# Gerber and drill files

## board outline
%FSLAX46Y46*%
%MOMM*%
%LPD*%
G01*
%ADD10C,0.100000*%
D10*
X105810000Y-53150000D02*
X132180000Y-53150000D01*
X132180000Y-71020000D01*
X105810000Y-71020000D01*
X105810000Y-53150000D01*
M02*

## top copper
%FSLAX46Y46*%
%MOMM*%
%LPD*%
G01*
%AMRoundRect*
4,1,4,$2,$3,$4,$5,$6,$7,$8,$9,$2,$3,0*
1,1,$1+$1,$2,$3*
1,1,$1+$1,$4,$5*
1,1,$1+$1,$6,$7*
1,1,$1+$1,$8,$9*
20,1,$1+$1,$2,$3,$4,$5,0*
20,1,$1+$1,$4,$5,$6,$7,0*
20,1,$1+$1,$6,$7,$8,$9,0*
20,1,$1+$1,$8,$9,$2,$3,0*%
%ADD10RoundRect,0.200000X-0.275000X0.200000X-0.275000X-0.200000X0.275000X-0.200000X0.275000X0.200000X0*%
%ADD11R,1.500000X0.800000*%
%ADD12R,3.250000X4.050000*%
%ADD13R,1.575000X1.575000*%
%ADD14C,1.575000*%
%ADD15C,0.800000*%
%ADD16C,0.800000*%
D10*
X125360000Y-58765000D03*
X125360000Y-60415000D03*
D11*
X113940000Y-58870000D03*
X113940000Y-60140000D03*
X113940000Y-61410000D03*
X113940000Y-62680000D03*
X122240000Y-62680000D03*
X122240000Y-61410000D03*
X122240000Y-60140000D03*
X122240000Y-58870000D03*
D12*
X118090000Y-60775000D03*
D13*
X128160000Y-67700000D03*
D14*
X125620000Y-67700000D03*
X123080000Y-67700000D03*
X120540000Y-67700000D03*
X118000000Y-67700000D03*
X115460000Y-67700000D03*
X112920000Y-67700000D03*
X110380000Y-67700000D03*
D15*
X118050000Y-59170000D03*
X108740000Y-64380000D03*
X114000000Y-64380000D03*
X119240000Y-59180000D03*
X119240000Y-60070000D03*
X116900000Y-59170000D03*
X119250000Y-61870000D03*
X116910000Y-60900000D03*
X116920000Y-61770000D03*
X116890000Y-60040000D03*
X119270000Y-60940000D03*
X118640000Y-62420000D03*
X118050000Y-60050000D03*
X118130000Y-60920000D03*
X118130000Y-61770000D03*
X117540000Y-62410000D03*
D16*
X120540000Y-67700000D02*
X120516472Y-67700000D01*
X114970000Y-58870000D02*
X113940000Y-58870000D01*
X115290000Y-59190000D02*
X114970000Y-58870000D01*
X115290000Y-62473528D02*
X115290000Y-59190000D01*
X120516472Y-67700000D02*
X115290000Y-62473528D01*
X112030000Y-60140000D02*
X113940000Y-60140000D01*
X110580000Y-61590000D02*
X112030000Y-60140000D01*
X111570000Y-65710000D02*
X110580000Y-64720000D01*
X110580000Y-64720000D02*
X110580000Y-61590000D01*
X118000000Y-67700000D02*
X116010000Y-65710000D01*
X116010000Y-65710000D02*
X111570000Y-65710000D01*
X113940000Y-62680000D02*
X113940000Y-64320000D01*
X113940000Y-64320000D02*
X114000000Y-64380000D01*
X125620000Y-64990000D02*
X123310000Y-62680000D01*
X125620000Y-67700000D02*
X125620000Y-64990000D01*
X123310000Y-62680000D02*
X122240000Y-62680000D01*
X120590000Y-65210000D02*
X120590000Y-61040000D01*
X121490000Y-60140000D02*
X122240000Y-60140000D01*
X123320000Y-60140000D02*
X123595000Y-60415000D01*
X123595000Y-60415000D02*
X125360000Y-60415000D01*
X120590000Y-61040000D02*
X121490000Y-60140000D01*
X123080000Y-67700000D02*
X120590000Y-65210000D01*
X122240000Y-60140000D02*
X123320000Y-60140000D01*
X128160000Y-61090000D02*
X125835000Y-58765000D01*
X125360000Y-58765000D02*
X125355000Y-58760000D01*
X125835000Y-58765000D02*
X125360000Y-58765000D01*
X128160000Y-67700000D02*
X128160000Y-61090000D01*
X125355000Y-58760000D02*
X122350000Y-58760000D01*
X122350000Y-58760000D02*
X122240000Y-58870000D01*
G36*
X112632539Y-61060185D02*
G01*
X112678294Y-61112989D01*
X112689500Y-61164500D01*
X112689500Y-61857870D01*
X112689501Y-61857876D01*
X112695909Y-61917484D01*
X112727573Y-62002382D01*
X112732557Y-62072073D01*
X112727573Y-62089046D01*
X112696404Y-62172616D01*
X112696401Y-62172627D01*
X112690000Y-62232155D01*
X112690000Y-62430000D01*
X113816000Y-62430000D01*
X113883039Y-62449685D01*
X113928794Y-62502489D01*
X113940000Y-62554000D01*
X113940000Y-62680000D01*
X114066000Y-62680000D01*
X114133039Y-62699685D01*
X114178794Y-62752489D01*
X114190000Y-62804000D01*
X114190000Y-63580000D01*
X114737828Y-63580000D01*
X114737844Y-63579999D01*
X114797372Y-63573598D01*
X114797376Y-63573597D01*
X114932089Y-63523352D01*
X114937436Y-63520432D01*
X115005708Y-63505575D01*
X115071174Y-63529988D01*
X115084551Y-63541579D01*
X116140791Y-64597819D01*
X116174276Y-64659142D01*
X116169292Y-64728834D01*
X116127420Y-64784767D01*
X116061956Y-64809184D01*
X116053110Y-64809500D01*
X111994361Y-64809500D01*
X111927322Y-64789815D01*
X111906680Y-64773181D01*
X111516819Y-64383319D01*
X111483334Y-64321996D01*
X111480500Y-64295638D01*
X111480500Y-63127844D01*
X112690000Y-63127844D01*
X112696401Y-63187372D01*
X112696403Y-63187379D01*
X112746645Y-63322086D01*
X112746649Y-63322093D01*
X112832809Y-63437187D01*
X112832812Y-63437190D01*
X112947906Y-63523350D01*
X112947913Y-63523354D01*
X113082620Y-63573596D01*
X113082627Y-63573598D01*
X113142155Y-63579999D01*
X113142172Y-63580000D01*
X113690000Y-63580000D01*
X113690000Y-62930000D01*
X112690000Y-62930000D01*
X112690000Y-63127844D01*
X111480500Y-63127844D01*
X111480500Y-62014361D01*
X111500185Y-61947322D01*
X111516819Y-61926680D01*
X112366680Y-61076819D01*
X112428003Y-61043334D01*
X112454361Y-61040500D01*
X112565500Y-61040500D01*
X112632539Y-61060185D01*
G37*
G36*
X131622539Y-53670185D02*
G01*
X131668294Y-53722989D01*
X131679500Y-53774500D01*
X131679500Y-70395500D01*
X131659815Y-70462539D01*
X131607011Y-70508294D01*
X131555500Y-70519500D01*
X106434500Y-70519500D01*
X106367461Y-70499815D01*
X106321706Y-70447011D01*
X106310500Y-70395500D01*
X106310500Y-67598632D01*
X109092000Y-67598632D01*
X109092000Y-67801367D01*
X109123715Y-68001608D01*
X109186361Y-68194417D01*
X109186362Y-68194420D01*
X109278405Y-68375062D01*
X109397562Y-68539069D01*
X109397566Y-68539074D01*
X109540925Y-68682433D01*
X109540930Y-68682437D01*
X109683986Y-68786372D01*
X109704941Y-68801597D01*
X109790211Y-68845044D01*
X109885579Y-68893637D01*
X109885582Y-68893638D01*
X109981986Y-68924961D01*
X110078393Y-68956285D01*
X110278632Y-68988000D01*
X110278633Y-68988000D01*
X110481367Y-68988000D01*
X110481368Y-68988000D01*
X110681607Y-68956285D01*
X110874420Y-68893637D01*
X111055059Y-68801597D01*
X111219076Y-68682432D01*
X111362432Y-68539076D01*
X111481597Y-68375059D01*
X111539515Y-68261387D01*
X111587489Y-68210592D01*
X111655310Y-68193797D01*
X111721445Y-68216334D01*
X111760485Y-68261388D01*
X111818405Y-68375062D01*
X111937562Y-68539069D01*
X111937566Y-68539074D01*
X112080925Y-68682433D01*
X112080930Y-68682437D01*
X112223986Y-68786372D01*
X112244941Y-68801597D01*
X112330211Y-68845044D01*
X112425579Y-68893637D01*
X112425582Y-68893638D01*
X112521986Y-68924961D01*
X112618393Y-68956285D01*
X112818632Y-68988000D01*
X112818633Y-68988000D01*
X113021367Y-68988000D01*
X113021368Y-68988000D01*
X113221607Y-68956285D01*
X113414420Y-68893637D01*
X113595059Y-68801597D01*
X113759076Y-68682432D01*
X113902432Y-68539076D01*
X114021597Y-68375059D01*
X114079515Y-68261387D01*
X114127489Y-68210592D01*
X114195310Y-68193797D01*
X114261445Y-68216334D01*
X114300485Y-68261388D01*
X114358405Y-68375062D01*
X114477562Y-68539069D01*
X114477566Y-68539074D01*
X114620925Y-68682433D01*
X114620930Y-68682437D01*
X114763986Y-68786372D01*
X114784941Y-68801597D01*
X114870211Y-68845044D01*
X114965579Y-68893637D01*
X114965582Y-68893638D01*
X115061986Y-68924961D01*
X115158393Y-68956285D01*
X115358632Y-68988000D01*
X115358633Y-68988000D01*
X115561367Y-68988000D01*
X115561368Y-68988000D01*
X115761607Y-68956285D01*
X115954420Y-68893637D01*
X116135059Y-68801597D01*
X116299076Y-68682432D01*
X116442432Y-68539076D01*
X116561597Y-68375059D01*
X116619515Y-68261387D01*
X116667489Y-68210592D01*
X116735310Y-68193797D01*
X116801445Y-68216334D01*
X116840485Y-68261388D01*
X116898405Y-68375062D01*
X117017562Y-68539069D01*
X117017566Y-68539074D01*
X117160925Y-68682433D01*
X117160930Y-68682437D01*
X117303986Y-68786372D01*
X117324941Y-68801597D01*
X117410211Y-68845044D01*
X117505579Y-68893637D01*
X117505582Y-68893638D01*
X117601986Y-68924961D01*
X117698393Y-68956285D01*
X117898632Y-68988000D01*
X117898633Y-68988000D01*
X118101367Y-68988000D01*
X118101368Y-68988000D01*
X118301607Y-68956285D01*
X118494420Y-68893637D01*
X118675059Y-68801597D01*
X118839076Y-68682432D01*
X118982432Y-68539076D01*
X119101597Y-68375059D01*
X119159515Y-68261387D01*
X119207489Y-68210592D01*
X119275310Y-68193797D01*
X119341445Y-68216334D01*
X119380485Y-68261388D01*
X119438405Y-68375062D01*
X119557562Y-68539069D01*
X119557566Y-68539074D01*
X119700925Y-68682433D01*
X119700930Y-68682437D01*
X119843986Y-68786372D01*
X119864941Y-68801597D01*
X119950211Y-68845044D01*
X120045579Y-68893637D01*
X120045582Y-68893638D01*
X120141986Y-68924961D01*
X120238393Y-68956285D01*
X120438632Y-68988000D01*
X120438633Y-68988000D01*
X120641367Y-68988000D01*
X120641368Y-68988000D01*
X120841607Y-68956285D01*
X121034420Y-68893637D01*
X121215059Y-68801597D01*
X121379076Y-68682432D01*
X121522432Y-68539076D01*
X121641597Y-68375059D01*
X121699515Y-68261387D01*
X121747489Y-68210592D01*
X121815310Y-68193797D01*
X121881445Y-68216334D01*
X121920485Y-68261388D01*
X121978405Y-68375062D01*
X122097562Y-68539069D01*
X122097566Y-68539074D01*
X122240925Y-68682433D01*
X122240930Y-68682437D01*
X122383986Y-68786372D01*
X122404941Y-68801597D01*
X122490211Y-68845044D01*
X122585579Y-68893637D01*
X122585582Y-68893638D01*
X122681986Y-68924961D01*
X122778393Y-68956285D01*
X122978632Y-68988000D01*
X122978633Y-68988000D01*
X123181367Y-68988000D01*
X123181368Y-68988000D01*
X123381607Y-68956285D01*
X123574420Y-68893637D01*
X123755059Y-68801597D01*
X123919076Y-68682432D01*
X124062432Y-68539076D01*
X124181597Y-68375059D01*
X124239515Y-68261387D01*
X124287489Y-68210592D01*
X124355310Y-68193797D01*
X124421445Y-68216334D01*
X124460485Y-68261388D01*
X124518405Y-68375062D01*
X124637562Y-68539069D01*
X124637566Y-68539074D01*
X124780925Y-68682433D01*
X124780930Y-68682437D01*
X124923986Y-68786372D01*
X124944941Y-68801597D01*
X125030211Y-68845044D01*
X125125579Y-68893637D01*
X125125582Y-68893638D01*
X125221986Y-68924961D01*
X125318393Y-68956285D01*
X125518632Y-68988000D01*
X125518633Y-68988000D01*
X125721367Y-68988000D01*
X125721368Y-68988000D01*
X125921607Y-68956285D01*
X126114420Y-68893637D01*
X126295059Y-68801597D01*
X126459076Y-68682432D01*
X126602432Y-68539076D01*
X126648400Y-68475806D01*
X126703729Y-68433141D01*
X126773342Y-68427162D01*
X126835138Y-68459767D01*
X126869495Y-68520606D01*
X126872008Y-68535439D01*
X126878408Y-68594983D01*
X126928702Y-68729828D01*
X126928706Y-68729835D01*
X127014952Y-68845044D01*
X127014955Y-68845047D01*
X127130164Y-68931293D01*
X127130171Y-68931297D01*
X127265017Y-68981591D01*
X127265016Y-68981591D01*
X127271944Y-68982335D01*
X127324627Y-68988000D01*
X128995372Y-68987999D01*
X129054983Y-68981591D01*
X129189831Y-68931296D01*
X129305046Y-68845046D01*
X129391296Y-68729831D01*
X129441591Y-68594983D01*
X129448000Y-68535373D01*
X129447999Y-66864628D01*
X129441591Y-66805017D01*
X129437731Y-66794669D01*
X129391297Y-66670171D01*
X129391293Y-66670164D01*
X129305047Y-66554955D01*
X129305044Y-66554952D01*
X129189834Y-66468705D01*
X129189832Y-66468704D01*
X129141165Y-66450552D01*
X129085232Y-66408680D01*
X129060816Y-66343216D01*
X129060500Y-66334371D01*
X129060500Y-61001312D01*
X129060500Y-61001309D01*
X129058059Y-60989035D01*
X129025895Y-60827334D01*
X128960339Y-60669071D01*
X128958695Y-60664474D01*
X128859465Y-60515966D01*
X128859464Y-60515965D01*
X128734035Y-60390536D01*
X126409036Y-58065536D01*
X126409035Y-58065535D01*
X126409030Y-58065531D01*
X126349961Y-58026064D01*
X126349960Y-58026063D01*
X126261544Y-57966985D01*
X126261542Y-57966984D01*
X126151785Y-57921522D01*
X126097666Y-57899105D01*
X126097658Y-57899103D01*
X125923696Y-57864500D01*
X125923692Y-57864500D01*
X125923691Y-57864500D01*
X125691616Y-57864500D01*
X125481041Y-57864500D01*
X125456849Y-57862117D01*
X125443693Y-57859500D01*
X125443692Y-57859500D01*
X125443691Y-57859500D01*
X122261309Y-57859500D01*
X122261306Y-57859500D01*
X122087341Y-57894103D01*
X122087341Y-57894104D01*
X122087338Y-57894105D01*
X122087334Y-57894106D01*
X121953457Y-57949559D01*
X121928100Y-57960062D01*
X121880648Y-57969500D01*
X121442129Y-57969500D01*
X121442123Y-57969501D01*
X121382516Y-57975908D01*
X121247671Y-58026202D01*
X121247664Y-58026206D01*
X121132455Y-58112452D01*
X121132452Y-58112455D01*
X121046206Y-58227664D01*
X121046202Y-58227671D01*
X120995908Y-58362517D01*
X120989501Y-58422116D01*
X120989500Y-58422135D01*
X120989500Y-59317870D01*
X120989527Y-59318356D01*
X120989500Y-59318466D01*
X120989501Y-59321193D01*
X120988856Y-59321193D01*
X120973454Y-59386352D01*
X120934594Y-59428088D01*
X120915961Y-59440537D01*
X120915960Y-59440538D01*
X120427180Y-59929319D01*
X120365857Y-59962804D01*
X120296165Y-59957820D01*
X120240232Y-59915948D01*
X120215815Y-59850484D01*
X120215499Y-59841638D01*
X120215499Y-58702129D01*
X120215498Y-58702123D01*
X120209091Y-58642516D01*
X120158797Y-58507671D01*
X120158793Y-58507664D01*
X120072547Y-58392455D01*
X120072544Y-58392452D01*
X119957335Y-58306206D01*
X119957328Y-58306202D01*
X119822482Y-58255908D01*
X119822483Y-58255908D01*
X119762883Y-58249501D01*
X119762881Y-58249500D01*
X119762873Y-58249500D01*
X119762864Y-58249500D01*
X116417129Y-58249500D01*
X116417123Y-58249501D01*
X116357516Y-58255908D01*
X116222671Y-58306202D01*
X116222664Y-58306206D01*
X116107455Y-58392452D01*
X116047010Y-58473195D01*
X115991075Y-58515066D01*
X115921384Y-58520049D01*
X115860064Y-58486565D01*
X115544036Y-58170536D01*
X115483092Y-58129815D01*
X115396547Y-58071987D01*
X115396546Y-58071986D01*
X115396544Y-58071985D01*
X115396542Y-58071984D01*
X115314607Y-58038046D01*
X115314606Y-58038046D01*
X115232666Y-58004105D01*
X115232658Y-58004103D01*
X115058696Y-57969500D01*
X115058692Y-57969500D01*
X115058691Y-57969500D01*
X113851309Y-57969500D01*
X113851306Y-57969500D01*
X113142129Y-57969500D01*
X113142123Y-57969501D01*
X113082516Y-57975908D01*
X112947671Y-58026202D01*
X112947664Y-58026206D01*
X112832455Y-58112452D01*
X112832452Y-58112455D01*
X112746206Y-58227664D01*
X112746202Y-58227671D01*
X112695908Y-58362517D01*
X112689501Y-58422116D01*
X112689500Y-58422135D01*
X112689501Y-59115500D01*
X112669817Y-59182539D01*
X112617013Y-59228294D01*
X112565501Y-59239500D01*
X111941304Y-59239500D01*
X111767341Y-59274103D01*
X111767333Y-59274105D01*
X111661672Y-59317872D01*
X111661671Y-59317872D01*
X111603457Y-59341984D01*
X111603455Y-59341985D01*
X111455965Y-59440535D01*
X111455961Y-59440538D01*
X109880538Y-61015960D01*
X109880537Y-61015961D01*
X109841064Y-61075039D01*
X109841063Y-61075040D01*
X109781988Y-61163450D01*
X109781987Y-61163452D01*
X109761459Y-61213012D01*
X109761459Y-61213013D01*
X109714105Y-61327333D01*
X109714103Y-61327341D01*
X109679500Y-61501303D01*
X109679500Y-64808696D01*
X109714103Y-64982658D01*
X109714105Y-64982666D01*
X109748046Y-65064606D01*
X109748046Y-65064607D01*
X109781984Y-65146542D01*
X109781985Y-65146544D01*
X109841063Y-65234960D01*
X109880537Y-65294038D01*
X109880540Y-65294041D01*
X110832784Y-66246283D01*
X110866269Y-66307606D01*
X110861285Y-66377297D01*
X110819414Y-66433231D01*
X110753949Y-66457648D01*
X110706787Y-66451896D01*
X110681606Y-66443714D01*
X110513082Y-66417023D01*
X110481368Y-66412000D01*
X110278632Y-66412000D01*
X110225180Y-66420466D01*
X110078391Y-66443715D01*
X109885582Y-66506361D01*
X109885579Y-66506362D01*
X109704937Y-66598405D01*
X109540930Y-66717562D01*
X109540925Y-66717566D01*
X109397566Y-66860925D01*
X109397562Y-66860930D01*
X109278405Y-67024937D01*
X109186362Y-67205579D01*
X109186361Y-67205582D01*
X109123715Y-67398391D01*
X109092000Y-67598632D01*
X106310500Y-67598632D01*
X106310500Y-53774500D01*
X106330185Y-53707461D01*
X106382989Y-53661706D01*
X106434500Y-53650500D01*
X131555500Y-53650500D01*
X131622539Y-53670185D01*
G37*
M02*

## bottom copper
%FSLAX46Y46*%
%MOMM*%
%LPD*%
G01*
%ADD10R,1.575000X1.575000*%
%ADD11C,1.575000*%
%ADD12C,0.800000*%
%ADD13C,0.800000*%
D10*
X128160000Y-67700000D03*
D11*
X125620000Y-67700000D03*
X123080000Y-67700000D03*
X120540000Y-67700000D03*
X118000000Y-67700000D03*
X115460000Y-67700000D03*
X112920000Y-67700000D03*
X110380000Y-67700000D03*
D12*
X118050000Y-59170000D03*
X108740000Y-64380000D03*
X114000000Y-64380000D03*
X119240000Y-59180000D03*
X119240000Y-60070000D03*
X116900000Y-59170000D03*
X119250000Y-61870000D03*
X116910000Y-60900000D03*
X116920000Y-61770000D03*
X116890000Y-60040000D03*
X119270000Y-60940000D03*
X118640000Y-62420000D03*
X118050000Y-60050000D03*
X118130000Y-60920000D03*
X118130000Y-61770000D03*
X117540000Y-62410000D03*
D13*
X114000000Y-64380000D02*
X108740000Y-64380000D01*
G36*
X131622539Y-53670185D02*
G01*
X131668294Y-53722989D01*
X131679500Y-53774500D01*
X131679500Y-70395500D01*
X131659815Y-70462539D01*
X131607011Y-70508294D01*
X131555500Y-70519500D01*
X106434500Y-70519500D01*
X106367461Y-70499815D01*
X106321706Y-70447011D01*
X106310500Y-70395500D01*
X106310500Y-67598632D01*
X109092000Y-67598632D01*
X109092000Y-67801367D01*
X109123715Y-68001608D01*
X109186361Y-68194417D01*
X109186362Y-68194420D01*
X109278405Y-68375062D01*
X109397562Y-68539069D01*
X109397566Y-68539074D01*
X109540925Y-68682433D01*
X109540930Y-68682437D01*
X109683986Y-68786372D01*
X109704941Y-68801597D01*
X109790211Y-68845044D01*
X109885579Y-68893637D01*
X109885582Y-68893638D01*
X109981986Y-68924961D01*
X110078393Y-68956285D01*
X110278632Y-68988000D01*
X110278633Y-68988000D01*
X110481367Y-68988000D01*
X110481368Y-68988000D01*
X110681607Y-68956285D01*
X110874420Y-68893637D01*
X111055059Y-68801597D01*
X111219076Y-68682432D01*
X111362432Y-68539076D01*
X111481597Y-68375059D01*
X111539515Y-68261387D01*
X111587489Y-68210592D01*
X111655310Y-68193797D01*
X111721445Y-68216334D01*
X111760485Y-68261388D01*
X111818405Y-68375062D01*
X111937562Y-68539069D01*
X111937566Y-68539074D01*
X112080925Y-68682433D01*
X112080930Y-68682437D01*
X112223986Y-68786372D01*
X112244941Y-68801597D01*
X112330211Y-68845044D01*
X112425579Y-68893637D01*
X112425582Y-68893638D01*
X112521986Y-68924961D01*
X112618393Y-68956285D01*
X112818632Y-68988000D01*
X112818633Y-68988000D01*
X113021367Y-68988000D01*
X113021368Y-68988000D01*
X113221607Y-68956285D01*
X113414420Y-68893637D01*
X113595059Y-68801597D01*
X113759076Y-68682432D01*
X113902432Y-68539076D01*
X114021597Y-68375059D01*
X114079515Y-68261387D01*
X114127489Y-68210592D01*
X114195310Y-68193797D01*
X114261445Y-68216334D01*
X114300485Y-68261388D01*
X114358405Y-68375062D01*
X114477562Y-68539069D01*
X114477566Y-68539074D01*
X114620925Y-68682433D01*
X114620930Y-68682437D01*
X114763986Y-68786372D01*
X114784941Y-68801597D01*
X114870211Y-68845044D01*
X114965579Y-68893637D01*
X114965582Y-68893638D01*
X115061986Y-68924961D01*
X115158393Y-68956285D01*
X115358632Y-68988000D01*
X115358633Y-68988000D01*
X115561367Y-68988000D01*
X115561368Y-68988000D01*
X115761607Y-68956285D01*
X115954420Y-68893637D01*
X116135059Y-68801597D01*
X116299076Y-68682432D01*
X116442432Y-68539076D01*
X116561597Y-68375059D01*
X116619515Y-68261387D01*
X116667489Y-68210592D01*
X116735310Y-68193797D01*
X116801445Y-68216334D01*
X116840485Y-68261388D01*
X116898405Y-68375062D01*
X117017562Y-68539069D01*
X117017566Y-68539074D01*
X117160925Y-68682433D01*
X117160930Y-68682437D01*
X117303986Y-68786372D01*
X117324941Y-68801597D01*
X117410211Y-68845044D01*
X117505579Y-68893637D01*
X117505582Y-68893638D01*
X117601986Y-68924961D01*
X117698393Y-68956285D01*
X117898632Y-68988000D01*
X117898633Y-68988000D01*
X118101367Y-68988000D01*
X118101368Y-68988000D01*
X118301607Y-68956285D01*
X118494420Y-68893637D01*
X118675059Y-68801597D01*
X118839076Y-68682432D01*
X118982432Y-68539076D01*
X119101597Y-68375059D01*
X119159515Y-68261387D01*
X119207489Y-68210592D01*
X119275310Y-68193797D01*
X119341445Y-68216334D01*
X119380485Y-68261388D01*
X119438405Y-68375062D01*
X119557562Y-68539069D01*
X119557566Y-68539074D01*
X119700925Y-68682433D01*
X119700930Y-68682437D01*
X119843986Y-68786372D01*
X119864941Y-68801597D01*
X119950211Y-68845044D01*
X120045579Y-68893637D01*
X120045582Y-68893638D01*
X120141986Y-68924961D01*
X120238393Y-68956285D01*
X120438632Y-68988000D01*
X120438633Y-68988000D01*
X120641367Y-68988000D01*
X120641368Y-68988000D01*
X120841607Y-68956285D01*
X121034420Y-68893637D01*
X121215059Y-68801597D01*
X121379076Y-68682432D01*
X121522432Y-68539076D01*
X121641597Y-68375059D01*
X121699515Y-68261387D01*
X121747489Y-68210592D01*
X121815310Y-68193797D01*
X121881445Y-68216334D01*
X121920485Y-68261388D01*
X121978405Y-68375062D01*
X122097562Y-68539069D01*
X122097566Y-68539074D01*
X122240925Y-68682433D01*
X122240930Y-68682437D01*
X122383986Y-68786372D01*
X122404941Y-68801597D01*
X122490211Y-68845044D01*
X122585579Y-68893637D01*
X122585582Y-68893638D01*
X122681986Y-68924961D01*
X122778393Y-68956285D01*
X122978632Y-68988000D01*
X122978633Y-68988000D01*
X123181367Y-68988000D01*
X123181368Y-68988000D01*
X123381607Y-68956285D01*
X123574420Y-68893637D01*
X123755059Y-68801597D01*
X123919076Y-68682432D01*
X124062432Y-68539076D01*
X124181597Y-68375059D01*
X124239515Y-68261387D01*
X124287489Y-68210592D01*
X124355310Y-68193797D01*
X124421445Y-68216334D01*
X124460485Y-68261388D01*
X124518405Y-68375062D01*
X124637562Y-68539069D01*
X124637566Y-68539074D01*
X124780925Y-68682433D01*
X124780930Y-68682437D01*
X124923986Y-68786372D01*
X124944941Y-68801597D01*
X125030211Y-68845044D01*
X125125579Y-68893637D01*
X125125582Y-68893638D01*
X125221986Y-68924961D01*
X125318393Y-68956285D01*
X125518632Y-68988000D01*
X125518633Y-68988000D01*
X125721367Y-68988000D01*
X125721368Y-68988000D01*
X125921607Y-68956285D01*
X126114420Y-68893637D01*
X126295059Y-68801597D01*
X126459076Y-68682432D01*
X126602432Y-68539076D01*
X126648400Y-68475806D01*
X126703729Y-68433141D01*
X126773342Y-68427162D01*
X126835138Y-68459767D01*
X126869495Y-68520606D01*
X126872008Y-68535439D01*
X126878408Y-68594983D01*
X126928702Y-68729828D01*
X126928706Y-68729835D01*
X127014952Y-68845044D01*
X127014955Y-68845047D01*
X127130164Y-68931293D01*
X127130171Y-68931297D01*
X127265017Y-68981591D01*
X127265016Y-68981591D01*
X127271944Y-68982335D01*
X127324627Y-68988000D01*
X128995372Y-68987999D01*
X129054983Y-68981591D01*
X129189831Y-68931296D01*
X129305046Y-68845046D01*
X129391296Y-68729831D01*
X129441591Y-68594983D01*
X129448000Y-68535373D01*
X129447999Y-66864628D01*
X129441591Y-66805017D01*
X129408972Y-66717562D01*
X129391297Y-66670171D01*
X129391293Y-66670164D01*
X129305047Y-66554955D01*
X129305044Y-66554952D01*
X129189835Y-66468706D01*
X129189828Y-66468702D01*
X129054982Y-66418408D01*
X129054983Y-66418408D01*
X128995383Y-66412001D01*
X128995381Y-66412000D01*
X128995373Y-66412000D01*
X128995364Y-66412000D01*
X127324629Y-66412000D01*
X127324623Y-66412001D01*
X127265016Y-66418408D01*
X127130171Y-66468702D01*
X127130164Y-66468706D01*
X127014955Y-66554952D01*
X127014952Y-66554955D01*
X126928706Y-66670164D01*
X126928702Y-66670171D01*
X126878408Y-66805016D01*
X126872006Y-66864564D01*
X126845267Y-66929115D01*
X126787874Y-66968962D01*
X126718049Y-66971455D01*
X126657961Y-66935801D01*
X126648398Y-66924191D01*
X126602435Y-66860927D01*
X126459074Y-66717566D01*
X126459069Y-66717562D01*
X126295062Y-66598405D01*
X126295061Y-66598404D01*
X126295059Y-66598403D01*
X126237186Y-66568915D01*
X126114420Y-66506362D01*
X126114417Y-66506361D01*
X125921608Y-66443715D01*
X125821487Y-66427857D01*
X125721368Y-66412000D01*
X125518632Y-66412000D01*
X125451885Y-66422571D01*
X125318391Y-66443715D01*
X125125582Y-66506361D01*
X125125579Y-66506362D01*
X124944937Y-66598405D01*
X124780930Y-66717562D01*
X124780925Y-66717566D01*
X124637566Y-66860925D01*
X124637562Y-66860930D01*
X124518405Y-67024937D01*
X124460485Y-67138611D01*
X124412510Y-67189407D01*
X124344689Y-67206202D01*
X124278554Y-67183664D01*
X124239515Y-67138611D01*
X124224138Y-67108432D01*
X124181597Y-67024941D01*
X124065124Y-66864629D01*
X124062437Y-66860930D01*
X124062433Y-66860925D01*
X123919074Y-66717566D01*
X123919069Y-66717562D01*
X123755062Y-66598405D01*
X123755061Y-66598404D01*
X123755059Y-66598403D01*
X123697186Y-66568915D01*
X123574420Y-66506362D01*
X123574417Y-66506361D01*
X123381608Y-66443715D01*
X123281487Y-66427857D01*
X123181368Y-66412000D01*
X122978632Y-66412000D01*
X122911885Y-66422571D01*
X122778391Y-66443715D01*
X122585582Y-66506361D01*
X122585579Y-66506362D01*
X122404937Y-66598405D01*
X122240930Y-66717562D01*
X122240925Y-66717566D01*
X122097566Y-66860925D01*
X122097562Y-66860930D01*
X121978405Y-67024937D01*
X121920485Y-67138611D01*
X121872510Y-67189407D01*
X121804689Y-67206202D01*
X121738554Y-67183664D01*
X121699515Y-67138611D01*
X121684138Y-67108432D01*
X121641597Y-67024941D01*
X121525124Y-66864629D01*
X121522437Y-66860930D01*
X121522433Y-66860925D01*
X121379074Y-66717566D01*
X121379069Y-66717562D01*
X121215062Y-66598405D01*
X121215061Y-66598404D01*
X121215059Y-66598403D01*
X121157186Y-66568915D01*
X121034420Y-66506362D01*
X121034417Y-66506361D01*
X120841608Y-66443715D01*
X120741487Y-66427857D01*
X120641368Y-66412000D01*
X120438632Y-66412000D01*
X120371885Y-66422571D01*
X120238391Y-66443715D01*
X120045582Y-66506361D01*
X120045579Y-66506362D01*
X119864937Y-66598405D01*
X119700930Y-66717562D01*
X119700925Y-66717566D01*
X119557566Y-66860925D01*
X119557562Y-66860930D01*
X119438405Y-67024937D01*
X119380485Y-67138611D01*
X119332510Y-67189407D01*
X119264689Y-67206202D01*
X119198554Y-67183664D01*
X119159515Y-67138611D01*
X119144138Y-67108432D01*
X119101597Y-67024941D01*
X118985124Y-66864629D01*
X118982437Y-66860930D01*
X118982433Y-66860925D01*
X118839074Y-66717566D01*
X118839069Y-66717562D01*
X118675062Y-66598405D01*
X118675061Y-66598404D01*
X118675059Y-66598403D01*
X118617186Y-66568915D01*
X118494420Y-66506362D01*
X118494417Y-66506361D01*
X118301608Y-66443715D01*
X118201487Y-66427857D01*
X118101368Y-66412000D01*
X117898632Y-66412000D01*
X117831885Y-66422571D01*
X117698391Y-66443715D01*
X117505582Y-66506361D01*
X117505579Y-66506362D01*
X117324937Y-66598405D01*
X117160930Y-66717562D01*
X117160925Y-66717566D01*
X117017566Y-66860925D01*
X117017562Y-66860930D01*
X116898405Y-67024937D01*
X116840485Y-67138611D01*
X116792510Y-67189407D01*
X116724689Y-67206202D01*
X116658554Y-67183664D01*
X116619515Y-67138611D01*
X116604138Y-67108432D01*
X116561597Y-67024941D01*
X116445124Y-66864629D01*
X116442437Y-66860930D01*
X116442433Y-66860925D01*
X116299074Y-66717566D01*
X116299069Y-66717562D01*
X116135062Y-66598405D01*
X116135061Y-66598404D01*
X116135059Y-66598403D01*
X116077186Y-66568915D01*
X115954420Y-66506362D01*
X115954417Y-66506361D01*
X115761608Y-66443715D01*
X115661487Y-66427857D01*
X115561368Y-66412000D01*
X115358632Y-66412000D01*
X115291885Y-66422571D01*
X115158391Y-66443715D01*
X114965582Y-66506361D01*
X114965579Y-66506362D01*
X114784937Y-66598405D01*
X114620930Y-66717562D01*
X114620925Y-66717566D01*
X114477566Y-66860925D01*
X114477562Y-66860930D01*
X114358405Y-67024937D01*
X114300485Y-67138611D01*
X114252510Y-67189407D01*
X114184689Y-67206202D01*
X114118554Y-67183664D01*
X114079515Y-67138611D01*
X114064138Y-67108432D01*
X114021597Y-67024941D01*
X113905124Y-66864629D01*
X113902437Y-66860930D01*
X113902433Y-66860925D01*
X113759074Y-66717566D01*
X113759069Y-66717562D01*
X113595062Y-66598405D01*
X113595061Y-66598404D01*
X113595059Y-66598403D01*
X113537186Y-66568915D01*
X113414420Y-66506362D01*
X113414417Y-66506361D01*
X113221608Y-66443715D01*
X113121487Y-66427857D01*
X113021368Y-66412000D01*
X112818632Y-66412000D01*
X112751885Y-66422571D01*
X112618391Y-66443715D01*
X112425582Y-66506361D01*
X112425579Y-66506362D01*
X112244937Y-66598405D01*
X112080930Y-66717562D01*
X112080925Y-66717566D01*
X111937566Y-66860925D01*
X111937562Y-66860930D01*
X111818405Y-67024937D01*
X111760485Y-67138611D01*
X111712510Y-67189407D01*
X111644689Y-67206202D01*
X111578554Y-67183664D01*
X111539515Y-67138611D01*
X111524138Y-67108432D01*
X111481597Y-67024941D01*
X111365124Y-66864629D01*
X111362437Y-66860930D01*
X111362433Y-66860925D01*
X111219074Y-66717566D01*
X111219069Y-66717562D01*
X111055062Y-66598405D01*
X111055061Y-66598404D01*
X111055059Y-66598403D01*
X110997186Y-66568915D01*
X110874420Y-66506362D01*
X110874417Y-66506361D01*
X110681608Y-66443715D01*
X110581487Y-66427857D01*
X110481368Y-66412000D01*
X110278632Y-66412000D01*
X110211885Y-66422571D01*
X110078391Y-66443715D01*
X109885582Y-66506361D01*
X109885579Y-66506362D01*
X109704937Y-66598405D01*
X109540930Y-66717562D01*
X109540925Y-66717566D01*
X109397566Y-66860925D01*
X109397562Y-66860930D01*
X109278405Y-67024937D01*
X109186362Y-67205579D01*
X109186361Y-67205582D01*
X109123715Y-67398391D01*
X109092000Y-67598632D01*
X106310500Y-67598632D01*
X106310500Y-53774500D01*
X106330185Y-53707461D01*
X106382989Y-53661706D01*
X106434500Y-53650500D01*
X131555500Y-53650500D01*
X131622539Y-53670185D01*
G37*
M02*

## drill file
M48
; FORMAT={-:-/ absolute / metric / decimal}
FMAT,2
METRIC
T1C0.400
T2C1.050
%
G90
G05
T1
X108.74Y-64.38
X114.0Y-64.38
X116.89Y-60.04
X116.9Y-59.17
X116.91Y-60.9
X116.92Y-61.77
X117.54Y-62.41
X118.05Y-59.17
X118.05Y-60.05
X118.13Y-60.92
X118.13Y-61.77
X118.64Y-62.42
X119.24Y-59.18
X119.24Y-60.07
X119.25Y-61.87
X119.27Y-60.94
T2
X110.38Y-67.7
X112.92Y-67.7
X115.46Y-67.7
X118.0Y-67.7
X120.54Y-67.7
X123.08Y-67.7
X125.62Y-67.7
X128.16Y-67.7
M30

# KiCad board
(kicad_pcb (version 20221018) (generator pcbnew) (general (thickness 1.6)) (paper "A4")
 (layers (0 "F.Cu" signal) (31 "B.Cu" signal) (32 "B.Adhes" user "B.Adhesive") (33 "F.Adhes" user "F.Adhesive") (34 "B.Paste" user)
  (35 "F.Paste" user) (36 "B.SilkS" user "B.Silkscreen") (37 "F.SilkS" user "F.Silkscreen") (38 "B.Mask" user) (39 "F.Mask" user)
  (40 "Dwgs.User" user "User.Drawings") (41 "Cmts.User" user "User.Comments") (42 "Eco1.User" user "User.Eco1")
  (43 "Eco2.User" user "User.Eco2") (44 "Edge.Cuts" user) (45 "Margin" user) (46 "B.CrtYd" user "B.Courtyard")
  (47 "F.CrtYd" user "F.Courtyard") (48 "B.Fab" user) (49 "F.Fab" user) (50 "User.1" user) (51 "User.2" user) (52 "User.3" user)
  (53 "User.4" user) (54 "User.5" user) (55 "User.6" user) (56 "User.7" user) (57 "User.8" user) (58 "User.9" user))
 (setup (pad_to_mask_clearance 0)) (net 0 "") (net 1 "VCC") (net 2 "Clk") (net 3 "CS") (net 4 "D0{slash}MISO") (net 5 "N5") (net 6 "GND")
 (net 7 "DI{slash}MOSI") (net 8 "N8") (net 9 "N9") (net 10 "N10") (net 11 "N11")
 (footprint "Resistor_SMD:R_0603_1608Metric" (layer "F.Cu") (at 125.36 59.59 -90)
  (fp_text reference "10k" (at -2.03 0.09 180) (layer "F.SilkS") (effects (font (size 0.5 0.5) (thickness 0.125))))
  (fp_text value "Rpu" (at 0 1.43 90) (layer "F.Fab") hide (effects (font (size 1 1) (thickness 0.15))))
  (pad "1" smd roundrect (at -0.825 0 270) (size 0.8 0.95) (layers "F.Cu" "F.Paste" "F.Mask") (roundrect_rratio 0.25) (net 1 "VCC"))
  (pad "2" smd roundrect (at 0.825 0 270) (size 0.8 0.95) (layers "F.Cu" "F.Paste" "F.Mask") (roundrect_rratio 0.25) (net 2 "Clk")))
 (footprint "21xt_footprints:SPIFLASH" (layer "F.Cu") (at 118.09 60.775)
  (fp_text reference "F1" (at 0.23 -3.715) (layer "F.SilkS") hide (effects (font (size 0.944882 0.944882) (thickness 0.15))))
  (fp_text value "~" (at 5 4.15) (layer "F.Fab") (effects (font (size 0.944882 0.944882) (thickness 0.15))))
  (pad "1" smd rect (at -4.15 -1.905) (size 1.5 0.8) (layers "F.Cu" "F.Mask") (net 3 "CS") (solder_mask_margin 0.102))
  (pad "2" smd rect (at -4.15 -0.635) (size 1.5 0.8) (layers "F.Cu" "F.Mask") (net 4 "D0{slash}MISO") (solder_mask_margin 0.102))
  (pad "3" smd rect (at -4.15 0.635) (size 1.5 0.8) (layers "F.Cu" "F.Mask") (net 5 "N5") (solder_mask_margin 0.102))
  (pad "4" smd rect (at -4.15 1.905) (size 1.5 0.8) (layers "F.Cu" "F.Mask") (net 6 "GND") (solder_mask_margin 0.102))
  (pad "5" smd rect (at 4.15 1.905) (size 1.5 0.8) (layers "F.Cu" "F.Mask") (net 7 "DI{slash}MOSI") (solder_mask_margin 0.102))
  (pad "6" smd rect (at 4.15 0.635) (size 1.5 0.8) (layers "F.Cu" "F.Mask") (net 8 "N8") (solder_mask_margin 0.102))
  (pad "7" smd rect (at 4.15 -0.635) (size 1.5 0.8) (layers "F.Cu" "F.Mask") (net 2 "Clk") (solder_mask_margin 0.102))
  (pad "8" smd rect (at 4.15 -1.905) (size 1.5 0.8) (layers "F.Cu" "F.Mask") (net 1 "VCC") (solder_mask_margin 0.102))
  (pad "9" smd rect (at 0 0) (size 3.25 4.05) (layers "F.Cu" "F.Mask") (solder_mask_margin 0.102)))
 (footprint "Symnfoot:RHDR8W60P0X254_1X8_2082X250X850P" (layer "F.Cu") (at 128.16 67.7 180)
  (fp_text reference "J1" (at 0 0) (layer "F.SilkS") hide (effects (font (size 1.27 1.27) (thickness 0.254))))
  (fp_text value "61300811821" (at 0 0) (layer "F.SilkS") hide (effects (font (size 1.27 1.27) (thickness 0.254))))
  (pad "1" thru_hole rect (at 0 0 180) (size 1.575 1.575) (drill 1.05) (layers "*.Cu" "*.Mask") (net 1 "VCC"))
  (pad "2" thru_hole circle (at 2.54 0 180) (size 1.575 1.575) (drill 1.05) (layers "*.Cu" "*.Mask") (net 7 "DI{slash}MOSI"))
  (pad "3" thru_hole circle (at 5.08 0 180) (size 1.575 1.575) (drill 1.05) (layers "*.Cu" "*.Mask") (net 2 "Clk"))
  (pad "4" thru_hole circle (at 7.62 0 180) (size 1.575 1.575) (drill 1.05) (layers "*.Cu" "*.Mask") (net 3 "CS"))
  (pad "5" thru_hole circle (at 10.16 0 180) (size 1.575 1.575) (drill 1.05) (layers "*.Cu" "*.Mask") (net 4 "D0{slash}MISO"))
  (pad "6" thru_hole circle (at 12.7 0 180) (size 1.575 1.575) (drill 1.05) (layers "*.Cu" "*.Mask") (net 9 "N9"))
  (pad "7" thru_hole circle (at 15.24 0 180) (size 1.575 1.575) (drill 1.05) (layers "*.Cu" "*.Mask") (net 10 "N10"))
  (pad "8" thru_hole circle (at 17.78 0 180) (size 1.575 1.575) (drill 1.05) (layers "*.Cu" "*.Mask") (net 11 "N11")))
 (gr_rect (start 105.81 53.15) (end 132.18 71.02) (stroke (width 0.1) (type default)) (fill none) (layer "Edge.Cuts"))
 (segment (start 120.54 67.7) (end 120.516472 67.7) (width 0.8) (layer "F.Cu") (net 3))
 (segment (start 114.97 58.87) (end 113.94 58.87) (width 0.8) (layer "F.Cu") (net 3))
 (segment (start 115.29 59.19) (end 114.97 58.87) (width 0.8) (layer "F.Cu") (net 3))
 (segment (start 115.29 62.473528) (end 115.29 59.19) (width 0.8) (layer "F.Cu") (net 3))
 (segment (start 120.516472 67.7) (end 115.29 62.473528) (width 0.8) (layer "F.Cu") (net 3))
 (segment (start 112.03 60.14) (end 113.94 60.14) (width 0.8) (layer "F.Cu") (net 4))
 (segment (start 110.58 61.59) (end 112.03 60.14) (width 0.8) (layer "F.Cu") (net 4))
 (segment (start 111.57 65.71) (end 110.58 64.72) (width 0.8) (layer "F.Cu") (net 4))
 (segment (start 110.58 64.72) (end 110.58 61.59) (width 0.8) (layer "F.Cu") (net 4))
 (segment (start 118 67.7) (end 116.01 65.71) (width 0.8) (layer "F.Cu") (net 4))
 (segment (start 116.01 65.71) (end 111.57 65.71) (width 0.8) (layer "F.Cu") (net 4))
 (segment (start 113.94 62.68) (end 113.94 64.32) (width 0.8) (layer "F.Cu") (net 6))
 (segment (start 113.94 64.32) (end 114 64.38) (width 0.8) (layer "F.Cu") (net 6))
 (via (at 118.05 59.17) (size 0.8) (drill 0.4) (layers "F.Cu" "B.Cu") (free) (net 6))
 (via (at 108.74 64.38) (size 0.8) (drill 0.4) (layers "F.Cu" "B.Cu") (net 6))
 (via (at 114 64.38) (size 0.8) (drill 0.4) (layers "F.Cu" "B.Cu") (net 6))
 (via (at 119.24 59.18) (size 0.8) (drill 0.4) (layers "F.Cu" "B.Cu") (free) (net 6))
 (via (at 119.24 60.07) (size 0.8) (drill 0.4) (layers "F.Cu" "B.Cu") (free) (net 6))
 (via (at 116.9 59.17) (size 0.8) (drill 0.4) (layers "F.Cu" "B.Cu") (free) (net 6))
 (via (at 119.25 61.87) (size 0.8) (drill 0.4) (layers "F.Cu" "B.Cu") (free) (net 6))
 (via (at 116.91 60.9) (size 0.8) (drill 0.4) (layers "F.Cu" "B.Cu") (free) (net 6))
 (via (at 116.92 61.77) (size 0.8) (drill 0.4) (layers "F.Cu" "B.Cu") (free) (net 6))
 (via (at 116.89 60.04) (size 0.8) (drill 0.4) (layers "F.Cu" "B.Cu") (free) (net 6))
 (via (at 119.27 60.94) (size 0.8) (drill 0.4) (layers "F.Cu" "B.Cu") (free) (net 6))
 (via (at 118.64 62.42) (size 0.8) (drill 0.4) (layers "F.Cu" "B.Cu") (free) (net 6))
 (via (at 118.05 60.05) (size 0.8) (drill 0.4) (layers "F.Cu" "B.Cu") (free) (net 6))
 (via (at 118.13 60.92) (size 0.8) (drill 0.4) (layers "F.Cu" "B.Cu") (free) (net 6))
 (via (at 118.13 61.77) (size 0.8) (drill 0.4) (layers "F.Cu" "B.Cu") (free) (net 6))
 (via (at 117.54 62.41) (size 0.8) (drill 0.4) (layers "F.Cu" "B.Cu") (free) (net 6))
 (segment (start 114 64.38) (end 108.74 64.38) (width 0.8) (layer "B.Cu") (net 6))
 (segment (start 125.62 64.99) (end 123.31 62.68) (width 0.8) (layer "F.Cu") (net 7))
 (segment (start 125.62 67.7) (end 125.62 64.99) (width 0.8) (layer "F.Cu") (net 7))
 (segment (start 123.31 62.68) (end 122.24 62.68) (width 0.8) (layer "F.Cu") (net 7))
 (segment (start 120.59 65.21) (end 120.59 61.04) (width 0.8) (layer "F.Cu") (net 2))
 (segment (start 121.49 60.14) (end 122.24 60.14) (width 0.8) (layer "F.Cu") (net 2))
 (segment (start 123.32 60.14) (end 123.595 60.415) (width 0.8) (layer "F.Cu") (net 2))
 (segment (start 123.595 60.415) (end 125.36 60.415) (width 0.8) (layer "F.Cu") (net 2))
 (segment (start 120.59 61.04) (end 121.49 60.14) (width 0.8) (layer "F.Cu") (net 2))
 (segment (start 123.08 67.7) (end 120.59 65.21) (width 0.8) (layer "F.Cu") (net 2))
 (segment (start 122.24 60.14) (end 123.32 60.14) (width 0.8) (layer "F.Cu") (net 2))
 (segment (start 128.16 61.09) (end 125.835 58.765) (width 0.8) (layer "F.Cu") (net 1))
 (segment (start 125.36 58.765) (end 125.355 58.76) (width 0.8) (layer "F.Cu") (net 1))
 (segment (start 125.835 58.765) (end 125.36 58.765) (width 0.8) (layer "F.Cu") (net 1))
 (segment (start 128.16 67.7) (end 128.16 61.09) (width 0.8) (layer "F.Cu") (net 1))
 (segment (start 125.355 58.76) (end 122.35 58.76) (width 0.8) (layer "F.Cu") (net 1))
 (segment (start 122.35 58.76) (end 122.24 58.87) (width 0.8) (layer "F.Cu") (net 1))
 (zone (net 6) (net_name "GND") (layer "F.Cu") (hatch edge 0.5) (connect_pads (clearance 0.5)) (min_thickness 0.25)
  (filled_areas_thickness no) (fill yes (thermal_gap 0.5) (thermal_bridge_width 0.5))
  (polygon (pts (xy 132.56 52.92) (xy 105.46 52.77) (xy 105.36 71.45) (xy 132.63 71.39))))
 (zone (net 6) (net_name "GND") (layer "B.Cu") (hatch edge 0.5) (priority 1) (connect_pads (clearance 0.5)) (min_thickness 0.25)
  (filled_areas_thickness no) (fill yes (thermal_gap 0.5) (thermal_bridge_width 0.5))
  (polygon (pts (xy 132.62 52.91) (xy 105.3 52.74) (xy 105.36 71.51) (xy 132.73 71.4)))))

